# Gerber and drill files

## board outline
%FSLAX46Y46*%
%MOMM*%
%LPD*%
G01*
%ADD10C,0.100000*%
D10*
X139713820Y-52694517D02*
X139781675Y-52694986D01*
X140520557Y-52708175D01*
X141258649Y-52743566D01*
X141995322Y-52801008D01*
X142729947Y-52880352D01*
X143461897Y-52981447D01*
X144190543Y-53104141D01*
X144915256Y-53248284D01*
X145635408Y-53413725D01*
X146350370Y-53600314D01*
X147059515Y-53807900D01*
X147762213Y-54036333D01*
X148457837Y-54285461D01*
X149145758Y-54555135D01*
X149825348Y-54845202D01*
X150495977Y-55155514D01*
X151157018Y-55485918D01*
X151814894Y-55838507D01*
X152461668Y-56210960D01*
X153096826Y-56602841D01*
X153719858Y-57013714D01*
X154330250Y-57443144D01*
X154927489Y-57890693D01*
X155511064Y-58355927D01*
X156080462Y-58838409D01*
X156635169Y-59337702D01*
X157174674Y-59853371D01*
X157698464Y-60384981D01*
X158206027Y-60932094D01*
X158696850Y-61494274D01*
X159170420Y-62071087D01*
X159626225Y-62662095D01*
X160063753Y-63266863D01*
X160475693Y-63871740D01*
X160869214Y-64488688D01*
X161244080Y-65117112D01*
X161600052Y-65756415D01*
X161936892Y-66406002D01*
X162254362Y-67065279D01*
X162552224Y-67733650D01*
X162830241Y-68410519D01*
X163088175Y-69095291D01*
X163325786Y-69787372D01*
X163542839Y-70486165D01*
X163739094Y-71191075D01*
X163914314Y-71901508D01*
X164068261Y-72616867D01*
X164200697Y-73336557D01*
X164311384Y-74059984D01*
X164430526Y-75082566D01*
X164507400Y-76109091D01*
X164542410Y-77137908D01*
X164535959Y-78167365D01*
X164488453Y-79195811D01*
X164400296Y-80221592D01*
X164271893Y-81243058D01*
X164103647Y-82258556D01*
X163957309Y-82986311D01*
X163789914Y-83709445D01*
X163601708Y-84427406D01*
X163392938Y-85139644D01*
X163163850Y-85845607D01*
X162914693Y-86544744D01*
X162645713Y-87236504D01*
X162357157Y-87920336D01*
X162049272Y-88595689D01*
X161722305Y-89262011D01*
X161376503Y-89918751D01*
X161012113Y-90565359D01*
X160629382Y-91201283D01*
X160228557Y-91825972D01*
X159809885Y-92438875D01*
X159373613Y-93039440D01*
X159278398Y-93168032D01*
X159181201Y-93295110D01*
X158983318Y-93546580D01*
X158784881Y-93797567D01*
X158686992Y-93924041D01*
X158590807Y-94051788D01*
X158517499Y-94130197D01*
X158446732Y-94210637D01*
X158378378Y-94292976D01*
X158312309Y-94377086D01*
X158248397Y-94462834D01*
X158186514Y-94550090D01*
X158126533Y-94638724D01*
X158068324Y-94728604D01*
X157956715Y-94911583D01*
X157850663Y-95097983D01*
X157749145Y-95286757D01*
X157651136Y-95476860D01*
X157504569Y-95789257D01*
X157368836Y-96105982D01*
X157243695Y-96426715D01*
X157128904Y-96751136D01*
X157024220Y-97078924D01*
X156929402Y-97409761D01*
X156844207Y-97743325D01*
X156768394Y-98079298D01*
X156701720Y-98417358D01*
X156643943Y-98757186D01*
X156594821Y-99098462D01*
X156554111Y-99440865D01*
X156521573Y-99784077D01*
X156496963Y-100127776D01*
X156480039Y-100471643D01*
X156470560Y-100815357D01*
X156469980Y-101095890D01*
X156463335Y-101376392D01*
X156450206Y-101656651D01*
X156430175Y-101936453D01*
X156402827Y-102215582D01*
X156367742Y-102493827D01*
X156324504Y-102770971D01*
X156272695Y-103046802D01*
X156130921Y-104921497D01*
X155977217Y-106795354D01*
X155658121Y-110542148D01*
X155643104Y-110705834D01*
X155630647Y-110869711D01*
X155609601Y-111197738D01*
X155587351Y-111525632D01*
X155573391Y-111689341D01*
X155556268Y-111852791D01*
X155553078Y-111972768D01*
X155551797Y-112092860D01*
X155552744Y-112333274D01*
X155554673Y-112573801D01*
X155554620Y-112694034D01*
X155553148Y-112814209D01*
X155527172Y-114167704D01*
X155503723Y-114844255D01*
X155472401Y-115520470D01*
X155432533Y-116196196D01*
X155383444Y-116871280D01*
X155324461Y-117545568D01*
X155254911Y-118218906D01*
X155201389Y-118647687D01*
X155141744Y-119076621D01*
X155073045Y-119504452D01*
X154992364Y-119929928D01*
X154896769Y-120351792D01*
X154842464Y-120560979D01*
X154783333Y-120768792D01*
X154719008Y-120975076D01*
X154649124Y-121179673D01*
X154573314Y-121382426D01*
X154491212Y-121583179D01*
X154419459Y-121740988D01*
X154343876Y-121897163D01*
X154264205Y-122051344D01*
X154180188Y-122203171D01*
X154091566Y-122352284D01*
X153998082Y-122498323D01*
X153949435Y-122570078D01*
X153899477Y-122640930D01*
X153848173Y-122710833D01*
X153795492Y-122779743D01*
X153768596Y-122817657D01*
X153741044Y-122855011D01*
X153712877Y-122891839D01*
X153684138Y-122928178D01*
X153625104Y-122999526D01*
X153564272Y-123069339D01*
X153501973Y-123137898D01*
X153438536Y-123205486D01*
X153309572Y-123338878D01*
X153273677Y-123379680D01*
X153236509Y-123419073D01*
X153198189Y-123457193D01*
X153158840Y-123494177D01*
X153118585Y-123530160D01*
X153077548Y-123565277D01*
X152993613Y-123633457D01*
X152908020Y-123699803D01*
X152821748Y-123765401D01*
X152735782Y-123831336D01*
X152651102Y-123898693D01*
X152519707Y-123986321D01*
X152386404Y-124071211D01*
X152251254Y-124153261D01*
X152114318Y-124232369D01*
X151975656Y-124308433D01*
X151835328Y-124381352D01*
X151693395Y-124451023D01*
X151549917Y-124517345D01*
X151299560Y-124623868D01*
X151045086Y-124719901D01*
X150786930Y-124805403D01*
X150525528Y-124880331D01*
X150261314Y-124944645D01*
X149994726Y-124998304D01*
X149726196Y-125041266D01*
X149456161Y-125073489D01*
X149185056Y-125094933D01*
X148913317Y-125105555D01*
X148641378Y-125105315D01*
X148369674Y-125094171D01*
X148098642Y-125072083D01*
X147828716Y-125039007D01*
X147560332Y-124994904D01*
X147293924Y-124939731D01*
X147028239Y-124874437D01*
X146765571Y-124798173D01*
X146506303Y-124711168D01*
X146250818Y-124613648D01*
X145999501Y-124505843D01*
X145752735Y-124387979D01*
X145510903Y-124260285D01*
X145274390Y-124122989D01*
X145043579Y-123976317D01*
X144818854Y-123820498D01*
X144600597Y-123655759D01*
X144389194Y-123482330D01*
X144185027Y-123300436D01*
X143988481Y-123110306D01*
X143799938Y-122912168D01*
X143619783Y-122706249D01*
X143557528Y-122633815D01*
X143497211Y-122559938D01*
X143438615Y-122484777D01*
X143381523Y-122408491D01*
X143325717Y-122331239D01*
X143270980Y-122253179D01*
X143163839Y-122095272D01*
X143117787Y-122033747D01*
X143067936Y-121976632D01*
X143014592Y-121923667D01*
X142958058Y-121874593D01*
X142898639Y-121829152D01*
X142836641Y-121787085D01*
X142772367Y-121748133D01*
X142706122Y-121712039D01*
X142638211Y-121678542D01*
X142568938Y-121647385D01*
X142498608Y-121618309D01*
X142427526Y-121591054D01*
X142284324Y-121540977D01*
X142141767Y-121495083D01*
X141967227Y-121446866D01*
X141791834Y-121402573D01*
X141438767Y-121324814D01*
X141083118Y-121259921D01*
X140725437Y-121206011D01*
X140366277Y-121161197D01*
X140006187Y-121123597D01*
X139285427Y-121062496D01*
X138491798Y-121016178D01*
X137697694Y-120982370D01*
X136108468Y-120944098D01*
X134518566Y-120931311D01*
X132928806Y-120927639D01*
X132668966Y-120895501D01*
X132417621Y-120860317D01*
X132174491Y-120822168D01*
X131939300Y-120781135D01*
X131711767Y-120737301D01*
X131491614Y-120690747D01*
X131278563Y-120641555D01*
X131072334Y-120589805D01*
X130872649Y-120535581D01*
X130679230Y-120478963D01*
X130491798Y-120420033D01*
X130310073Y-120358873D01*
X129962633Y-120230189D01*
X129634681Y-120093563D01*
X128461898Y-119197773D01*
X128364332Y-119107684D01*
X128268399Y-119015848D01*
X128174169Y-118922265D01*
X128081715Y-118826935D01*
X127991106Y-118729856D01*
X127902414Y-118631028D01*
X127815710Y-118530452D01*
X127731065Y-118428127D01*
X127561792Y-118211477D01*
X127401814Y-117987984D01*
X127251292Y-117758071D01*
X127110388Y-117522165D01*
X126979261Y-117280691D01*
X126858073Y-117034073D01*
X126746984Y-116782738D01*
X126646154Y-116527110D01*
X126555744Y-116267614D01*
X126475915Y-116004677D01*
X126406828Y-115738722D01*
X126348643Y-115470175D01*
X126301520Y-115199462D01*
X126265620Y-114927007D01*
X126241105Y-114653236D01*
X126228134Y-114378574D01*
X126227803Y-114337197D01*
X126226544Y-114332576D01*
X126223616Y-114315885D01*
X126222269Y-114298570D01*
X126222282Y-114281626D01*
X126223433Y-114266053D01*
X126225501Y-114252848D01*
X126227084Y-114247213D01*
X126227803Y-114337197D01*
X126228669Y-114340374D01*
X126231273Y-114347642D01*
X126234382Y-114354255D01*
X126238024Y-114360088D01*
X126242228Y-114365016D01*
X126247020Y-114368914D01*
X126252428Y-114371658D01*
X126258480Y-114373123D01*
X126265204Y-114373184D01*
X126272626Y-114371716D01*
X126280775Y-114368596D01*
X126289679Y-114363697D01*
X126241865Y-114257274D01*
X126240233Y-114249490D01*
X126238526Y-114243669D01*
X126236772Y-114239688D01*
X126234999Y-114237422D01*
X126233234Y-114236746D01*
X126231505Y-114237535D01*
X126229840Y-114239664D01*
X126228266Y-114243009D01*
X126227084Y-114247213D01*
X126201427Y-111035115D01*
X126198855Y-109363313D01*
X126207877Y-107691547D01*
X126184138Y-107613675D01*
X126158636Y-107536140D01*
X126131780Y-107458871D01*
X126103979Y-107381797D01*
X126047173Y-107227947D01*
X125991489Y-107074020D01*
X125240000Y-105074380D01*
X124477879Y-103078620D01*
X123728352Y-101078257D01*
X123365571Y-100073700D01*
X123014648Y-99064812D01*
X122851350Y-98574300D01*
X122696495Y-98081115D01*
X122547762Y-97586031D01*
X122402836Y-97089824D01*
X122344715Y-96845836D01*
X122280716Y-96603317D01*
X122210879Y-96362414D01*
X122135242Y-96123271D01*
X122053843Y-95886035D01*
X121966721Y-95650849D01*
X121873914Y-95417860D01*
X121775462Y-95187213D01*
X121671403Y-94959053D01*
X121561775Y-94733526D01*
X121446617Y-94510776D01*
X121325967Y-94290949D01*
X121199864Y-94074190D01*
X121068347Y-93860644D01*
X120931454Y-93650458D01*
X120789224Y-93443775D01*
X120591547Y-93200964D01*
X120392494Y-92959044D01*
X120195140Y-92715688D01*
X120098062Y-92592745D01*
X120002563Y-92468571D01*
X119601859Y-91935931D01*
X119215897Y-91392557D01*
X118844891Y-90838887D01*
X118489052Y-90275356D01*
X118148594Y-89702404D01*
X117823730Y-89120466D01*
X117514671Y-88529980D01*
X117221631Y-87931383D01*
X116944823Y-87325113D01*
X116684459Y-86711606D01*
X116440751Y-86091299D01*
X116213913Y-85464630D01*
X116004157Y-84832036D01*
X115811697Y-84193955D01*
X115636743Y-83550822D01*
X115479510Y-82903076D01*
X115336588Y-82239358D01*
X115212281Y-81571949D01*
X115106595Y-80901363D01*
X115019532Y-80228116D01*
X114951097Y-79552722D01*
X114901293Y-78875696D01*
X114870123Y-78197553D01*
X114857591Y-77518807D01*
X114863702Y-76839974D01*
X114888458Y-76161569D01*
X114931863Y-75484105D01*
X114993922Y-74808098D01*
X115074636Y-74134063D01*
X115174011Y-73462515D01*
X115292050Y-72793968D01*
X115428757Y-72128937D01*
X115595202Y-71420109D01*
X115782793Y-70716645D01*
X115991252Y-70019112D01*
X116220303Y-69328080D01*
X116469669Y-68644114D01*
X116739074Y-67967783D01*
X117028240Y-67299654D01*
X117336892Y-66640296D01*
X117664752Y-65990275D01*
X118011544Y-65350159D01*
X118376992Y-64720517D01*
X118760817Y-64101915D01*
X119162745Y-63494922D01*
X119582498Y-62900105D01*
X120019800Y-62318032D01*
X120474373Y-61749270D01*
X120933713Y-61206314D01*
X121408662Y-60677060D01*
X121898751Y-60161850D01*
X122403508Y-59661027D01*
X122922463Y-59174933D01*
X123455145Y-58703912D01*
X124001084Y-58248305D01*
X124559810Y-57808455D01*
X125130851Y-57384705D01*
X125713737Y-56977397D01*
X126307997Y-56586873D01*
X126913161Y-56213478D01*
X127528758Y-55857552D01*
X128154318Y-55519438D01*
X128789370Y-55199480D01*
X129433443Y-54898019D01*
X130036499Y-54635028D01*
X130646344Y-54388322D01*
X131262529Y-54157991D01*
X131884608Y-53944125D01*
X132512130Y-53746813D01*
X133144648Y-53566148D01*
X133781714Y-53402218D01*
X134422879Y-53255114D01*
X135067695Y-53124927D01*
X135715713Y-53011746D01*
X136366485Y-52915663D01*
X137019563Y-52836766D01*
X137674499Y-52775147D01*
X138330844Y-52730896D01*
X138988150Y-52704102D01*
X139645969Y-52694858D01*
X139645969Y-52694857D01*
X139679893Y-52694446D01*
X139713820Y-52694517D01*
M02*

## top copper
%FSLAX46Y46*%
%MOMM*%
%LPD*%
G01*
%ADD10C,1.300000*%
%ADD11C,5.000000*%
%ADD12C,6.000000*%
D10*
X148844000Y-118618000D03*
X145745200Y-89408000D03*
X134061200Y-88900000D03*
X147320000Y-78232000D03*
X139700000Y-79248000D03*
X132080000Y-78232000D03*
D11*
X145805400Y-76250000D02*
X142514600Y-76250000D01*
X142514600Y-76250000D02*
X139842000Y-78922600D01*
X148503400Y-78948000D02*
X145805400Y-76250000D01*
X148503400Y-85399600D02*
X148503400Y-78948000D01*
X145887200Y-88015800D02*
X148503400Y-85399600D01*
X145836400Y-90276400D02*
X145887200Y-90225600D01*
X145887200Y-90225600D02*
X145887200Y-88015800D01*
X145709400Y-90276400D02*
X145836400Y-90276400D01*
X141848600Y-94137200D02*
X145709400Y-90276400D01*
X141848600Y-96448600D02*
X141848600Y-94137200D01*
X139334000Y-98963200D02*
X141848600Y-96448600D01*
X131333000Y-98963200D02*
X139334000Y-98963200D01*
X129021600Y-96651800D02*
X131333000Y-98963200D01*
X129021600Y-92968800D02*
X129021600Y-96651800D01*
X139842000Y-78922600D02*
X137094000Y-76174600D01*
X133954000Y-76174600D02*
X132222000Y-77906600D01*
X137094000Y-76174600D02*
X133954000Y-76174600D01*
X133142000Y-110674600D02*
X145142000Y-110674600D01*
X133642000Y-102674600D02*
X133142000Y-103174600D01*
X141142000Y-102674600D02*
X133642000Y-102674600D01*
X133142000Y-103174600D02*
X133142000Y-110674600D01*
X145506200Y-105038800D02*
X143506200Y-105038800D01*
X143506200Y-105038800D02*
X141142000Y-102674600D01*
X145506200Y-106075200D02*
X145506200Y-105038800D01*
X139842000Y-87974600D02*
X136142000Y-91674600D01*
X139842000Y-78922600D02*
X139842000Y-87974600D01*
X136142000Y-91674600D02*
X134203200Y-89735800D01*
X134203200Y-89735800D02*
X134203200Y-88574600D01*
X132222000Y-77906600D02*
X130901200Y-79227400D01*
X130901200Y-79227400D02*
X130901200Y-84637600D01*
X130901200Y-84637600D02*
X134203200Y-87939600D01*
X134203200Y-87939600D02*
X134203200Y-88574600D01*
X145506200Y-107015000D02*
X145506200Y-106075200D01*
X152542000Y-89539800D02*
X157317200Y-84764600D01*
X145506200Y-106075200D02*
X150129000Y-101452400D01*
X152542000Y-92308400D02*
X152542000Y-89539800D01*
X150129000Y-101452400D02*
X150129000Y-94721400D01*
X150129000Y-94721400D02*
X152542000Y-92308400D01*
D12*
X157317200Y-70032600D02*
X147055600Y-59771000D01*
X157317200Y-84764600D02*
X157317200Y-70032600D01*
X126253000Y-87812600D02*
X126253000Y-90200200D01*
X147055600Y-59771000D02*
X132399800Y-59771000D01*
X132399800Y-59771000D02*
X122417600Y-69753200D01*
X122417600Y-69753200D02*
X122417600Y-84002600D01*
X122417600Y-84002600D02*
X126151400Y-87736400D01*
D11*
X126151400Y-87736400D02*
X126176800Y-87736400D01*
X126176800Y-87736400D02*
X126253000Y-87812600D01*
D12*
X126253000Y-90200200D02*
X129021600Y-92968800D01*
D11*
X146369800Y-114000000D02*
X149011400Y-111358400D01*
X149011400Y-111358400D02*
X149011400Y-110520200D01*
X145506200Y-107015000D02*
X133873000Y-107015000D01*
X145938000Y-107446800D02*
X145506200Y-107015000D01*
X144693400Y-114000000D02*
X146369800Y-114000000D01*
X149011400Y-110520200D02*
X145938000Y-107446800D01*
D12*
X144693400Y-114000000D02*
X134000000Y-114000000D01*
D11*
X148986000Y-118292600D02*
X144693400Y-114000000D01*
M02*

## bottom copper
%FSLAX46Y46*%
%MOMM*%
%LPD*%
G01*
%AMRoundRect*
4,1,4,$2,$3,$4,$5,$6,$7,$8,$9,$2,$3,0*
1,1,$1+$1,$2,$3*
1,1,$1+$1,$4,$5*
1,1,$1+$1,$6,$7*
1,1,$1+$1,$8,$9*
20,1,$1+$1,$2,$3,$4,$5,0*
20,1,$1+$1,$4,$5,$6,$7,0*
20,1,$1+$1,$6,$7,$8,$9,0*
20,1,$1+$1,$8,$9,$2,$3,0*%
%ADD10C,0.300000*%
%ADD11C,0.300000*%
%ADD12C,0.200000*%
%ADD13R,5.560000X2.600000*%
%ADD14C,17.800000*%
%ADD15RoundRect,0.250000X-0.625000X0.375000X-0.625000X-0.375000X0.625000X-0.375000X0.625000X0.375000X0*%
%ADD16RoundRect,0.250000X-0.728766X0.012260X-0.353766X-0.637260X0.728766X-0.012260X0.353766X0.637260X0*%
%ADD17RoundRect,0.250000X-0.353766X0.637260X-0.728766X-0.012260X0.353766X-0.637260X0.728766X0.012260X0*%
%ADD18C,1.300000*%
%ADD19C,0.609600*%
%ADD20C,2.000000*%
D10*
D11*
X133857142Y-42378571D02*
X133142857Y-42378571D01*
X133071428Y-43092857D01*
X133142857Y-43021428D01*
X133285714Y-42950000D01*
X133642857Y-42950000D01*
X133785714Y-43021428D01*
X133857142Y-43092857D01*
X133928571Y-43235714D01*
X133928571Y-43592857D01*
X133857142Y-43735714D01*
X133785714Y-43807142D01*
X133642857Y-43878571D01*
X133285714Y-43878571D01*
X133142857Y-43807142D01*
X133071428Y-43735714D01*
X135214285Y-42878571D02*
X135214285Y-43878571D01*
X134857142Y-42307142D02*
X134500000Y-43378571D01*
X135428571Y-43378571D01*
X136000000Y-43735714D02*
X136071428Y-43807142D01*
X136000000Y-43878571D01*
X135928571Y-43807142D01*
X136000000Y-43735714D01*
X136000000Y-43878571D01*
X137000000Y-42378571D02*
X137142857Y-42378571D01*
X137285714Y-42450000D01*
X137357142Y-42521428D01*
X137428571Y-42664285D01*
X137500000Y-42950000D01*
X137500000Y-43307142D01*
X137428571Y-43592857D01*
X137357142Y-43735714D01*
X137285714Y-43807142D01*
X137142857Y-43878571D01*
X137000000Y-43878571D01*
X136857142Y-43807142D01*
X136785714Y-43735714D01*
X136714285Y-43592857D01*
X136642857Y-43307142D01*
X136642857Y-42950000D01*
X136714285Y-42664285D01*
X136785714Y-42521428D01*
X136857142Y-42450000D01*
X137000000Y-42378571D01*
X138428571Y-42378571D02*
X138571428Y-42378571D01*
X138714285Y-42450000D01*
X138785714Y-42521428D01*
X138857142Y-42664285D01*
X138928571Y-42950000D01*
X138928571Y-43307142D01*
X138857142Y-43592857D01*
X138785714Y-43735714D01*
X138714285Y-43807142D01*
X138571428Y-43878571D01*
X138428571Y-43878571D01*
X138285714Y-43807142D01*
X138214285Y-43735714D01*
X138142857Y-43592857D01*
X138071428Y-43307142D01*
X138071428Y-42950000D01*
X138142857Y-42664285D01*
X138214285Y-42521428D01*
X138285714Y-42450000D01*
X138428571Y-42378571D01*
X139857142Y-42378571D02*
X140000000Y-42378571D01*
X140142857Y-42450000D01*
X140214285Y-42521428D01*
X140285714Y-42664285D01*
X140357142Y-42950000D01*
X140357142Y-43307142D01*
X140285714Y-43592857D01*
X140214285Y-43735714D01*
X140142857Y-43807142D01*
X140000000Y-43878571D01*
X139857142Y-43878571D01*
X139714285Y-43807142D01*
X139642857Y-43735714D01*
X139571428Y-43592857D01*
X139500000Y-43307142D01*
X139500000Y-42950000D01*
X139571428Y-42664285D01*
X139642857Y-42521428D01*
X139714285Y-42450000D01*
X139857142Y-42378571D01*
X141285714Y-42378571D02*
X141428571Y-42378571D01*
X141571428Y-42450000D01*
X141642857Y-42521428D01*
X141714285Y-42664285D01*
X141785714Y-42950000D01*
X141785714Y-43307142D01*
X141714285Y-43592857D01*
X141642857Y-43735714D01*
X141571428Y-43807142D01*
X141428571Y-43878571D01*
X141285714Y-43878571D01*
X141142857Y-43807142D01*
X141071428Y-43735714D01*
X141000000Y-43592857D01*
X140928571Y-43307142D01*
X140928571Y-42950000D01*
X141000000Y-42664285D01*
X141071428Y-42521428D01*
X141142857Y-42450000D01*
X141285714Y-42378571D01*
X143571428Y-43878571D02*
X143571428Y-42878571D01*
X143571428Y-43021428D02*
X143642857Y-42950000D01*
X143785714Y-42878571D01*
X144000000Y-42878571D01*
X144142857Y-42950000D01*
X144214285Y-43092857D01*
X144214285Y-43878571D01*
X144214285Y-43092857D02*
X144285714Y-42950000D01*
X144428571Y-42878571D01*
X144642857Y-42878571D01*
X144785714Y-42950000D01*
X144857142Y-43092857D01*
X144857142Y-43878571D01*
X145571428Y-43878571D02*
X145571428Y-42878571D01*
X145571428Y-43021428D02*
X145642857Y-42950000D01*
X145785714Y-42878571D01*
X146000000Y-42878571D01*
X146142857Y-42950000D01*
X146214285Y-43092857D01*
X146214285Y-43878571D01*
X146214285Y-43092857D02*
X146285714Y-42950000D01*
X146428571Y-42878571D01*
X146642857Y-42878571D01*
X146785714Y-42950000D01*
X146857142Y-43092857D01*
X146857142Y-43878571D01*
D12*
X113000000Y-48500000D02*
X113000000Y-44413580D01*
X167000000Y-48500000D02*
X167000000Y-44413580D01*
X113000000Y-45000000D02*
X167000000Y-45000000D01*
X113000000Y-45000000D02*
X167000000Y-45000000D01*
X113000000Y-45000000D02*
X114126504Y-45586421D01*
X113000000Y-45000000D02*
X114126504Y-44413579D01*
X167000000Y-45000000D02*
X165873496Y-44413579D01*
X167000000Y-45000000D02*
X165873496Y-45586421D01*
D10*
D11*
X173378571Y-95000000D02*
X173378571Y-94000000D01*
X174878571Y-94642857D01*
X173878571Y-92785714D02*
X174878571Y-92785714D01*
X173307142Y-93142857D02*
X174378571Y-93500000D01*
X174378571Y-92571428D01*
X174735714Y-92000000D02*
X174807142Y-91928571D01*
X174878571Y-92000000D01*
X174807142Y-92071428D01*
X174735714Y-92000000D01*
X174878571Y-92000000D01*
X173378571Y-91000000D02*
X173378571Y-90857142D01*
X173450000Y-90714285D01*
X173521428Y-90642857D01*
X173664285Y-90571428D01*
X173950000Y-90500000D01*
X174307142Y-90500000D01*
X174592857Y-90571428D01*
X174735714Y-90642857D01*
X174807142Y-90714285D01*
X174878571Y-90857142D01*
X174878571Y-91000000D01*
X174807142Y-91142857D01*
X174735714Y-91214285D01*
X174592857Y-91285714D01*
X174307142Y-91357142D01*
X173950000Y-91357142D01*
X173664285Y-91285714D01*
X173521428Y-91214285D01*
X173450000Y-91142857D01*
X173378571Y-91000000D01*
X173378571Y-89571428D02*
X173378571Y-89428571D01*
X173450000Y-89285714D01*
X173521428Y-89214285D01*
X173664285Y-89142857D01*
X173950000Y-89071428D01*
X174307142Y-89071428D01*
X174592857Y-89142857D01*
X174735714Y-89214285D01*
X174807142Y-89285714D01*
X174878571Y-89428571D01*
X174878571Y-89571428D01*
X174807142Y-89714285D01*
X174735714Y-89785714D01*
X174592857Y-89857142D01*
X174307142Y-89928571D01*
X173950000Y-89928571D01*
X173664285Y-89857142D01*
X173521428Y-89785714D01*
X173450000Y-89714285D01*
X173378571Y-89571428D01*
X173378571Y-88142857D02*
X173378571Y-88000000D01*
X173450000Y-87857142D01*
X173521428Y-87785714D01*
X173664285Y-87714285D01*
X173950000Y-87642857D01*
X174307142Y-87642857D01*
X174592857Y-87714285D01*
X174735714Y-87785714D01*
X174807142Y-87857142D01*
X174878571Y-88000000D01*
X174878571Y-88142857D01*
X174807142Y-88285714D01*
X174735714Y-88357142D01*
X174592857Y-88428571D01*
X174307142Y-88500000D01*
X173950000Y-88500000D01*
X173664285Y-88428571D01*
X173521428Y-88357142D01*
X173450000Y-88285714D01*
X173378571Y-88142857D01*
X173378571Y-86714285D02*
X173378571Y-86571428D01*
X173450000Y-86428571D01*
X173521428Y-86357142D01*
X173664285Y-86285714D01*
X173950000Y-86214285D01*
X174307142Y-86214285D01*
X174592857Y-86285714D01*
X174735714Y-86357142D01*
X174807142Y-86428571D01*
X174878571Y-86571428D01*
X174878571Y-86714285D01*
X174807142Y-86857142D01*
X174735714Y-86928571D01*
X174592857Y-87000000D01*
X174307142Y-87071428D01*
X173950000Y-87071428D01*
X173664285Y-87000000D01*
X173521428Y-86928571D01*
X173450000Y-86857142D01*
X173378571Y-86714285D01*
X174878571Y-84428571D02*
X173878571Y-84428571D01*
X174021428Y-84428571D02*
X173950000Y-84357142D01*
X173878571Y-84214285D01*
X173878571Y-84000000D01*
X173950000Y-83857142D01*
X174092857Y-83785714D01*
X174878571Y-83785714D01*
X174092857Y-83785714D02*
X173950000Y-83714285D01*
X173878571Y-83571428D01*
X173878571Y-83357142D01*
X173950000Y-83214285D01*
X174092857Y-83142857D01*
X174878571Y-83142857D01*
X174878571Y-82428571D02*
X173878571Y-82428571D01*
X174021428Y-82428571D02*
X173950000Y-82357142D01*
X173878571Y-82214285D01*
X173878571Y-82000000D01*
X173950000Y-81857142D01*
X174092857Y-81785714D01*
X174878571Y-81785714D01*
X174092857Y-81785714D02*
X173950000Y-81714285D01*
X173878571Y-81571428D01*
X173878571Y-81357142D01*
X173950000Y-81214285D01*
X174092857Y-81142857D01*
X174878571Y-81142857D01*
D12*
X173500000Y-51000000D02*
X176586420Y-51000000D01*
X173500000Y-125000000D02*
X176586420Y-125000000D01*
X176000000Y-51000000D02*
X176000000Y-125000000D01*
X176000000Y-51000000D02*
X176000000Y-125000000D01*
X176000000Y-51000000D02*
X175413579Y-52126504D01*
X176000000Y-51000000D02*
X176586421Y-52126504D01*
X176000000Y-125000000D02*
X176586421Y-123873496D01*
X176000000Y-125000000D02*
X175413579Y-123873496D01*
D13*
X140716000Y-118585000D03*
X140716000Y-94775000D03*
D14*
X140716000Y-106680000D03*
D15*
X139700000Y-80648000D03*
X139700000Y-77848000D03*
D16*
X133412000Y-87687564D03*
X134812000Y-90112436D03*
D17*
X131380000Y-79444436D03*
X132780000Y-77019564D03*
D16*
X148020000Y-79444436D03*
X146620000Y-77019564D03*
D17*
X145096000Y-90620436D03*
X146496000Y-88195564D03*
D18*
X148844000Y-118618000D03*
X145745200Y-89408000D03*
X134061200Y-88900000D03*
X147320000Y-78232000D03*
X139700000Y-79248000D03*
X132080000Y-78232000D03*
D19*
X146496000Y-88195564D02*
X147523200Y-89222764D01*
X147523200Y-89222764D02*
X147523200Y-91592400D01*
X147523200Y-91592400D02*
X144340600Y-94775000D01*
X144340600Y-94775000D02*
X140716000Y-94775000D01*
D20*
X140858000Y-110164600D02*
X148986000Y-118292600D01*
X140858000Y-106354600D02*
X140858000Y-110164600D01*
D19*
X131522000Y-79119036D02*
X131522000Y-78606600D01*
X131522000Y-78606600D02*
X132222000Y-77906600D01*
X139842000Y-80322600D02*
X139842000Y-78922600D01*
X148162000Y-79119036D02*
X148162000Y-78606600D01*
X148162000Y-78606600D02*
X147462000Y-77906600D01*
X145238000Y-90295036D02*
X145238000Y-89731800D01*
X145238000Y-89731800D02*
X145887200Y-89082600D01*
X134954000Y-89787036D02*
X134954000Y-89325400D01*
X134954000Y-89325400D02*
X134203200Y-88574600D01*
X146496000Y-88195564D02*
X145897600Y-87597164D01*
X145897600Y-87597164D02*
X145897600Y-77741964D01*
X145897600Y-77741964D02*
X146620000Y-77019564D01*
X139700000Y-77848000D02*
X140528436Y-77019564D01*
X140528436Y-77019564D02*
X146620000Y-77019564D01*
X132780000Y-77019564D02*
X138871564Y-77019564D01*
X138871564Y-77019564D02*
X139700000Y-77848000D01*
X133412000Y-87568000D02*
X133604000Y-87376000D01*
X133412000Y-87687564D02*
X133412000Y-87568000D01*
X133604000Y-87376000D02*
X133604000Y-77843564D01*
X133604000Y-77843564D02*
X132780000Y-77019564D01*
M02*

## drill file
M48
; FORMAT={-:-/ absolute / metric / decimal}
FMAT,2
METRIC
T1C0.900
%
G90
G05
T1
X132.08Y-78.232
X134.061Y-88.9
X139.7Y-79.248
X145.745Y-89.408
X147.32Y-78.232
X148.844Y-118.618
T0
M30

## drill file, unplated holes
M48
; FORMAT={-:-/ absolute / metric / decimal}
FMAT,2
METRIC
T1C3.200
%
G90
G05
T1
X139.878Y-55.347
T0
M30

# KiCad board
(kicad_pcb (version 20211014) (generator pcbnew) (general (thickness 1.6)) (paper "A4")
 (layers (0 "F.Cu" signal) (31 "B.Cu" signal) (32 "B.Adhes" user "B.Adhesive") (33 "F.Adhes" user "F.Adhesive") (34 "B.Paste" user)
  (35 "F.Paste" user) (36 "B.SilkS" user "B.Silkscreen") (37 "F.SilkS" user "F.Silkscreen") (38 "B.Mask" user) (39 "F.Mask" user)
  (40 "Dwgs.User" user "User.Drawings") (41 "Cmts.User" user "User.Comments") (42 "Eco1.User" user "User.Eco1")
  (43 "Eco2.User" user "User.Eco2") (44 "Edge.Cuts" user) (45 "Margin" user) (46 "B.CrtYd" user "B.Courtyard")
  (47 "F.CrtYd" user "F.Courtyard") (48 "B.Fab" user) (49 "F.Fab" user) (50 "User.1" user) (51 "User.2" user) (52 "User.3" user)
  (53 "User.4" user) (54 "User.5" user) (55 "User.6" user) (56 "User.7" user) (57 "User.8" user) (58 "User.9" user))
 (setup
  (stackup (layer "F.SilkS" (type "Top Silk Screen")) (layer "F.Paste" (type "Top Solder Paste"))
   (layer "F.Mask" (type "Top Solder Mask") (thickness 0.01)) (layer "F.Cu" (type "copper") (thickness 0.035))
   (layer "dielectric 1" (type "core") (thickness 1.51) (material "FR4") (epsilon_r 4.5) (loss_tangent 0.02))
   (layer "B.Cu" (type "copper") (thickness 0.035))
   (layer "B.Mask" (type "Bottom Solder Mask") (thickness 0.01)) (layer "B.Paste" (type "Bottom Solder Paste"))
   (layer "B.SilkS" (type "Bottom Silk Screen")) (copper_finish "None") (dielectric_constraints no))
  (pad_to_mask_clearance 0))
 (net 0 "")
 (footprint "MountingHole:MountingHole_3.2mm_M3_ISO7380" (layer "F.Cu") (at 139.8778 55.3466)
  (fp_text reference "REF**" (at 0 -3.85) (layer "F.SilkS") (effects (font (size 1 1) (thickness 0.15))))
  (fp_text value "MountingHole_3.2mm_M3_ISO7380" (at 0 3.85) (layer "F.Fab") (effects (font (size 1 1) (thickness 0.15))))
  (pad "" np_thru_hole circle (at 0 0) (size 3.2 3.2) (drill 3.2) (layers *.Cu *.Mask)))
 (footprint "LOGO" (layer "F.Cu") (at 139.7 88.9)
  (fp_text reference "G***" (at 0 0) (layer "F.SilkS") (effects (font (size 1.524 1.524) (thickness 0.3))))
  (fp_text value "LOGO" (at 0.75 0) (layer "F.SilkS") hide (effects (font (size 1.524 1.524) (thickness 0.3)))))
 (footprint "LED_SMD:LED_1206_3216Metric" (layer "B.Cu") (at 139.7 79.248 -90)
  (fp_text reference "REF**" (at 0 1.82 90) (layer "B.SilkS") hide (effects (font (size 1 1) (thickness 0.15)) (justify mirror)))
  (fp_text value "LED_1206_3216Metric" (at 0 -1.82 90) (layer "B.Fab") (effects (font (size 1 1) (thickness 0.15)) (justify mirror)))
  (pad "1" smd roundrect (at -1.4 0 270) (size 1.25 1.75) (layers "B.Cu" "B.Paste" "B.Mask") (roundrect_rratio 0.2))
  (pad "2" smd roundrect (at 1.4 0 270) (size 1.25 1.75) (layers "B.Cu" "B.Paste" "B.Mask") (roundrect_rratio 0.2)))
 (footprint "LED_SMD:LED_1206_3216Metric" (layer "B.Cu") (at 147.32 78.232 -60)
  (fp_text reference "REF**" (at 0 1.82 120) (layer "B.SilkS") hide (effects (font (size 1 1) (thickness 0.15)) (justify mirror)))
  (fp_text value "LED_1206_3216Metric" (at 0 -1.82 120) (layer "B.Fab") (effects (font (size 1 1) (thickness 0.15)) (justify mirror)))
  (pad "1" smd roundrect (at -1.4 0 300) (size 1.25 1.75) (layers "B.Cu" "B.Paste" "B.Mask") (roundrect_rratio 0.2))
  (pad "2" smd roundrect (at 1.4 0 300) (size 1.25 1.75) (layers "B.Cu" "B.Paste" "B.Mask") (roundrect_rratio 0.2)))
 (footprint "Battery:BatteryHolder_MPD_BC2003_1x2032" (layer "B.Cu") (at 140.716 106.68 90)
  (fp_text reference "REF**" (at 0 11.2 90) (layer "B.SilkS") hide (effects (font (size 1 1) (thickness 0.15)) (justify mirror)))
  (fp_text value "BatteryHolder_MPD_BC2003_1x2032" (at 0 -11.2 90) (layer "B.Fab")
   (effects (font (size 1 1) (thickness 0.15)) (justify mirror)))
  (pad "1" smd rect (at 11.905 0 90) (size 2.6 5.56) (layers "B.Cu" "B.Paste" "B.Mask"))
  (pad "1" smd rect (at -11.905 0 90) (size 2.6 5.56) (layers "B.Cu" "B.Paste" "B.Mask"))
  (pad "2" smd circle (at 0 0 90) (size 17.8 17.8) (layers "B.Cu" "B.Mask")))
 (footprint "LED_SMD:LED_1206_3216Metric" (layer "B.Cu") (at 132.08 78.232 -120)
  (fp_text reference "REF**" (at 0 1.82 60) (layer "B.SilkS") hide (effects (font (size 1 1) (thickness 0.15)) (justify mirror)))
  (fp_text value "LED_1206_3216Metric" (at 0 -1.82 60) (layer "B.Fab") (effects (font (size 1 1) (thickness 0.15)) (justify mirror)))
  (pad "1" smd roundrect (at -1.4 0 240) (size 1.25 1.75) (layers "B.Cu" "B.Paste" "B.Mask") (roundrect_rratio 0.2))
  (pad "2" smd roundrect (at 1.4 0 240) (size 1.25 1.75) (layers "B.Cu" "B.Paste" "B.Mask") (roundrect_rratio 0.2)))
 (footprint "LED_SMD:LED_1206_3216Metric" (layer "B.Cu") (at 134.112 88.9 -60)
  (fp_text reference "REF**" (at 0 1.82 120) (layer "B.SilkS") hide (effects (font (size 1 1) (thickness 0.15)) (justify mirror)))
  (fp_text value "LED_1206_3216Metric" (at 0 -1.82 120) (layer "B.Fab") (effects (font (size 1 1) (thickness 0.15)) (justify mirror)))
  (pad "1" smd roundrect (at -1.4 0 300) (size 1.25 1.75) (layers "B.Cu" "B.Paste" "B.Mask") (roundrect_rratio 0.2))
  (pad "2" smd roundrect (at 1.4 0 300) (size 1.25 1.75) (layers "B.Cu" "B.Paste" "B.Mask") (roundrect_rratio 0.2)))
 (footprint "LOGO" (layer "B.Cu") (at 139.7 88.9 180)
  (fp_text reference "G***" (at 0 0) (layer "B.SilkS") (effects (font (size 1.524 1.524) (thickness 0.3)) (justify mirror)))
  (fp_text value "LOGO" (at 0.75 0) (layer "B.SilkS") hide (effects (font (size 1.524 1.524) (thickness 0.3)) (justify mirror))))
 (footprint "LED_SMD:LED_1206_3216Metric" (layer "B.Cu") (at 145.796 89.408 -120)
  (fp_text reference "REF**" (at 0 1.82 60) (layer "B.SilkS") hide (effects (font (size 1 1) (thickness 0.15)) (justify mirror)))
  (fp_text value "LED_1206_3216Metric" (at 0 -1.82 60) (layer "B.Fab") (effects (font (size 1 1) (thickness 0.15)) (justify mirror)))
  (pad "1" smd roundrect (at -1.4 0 240) (size 1.25 1.75) (layers "B.Cu" "B.Paste" "B.Mask") (roundrect_rratio 0.2))
  (pad "2" smd roundrect (at 1.4 0 240) (size 1.25 1.75) (layers "B.Cu" "B.Paste" "B.Mask") (roundrect_rratio 0.2)))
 (gr_poly
  (pts (xy 139.71382 52.694517) (xy 139.781675 52.694986) (xy 140.520557 52.708175) (xy 141.258649 52.743566) (xy 141.995322 52.801008)
   (xy 142.729947 52.880352) (xy 143.461897 52.981447) (xy 144.190543 53.104141) (xy 144.915256 53.248284) (xy 145.635408 53.413725)
   (xy 146.35037 53.600314) (xy 147.059515 53.8079) (xy 147.762213 54.036333) (xy 148.457837 54.285461) (xy 149.145758 54.555135)
   (xy 149.825348 54.845202) (xy 150.495977 55.155514) (xy 151.157018 55.485918) (xy 151.814894 55.838507) (xy 152.461668 56.21096)
   (xy 153.096826 56.602841) (xy 153.719858 57.013714) (xy 154.33025 57.443144) (xy 154.927489 57.890693) (xy 155.511064 58.355927)
   (xy 156.080462 58.838409) (xy 156.635169 59.337702) (xy 157.174674 59.853371) (xy 157.698464 60.384981) (xy 158.206027 60.932094)
   (xy 158.69685 61.494274) (xy 159.17042 62.071087) (xy 159.626225 62.662095) (xy 160.063753 63.266863) (xy 160.475693 63.87174)
   (xy 160.869214 64.488688) (xy 161.24408 65.117112) (xy 161.600052 65.756415) (xy 161.936892 66.406002) (xy 162.254362 67.065279)
   (xy 162.552224 67.73365) (xy 162.830241 68.410519) (xy 163.088175 69.095291) (xy 163.325786 69.787372) (xy 163.542839 70.486165)
   (xy 163.739094 71.191075) (xy 163.914314 71.901508) (xy 164.068261 72.616867) (xy 164.200697 73.336557) (xy 164.311384 74.059984)
   (xy 164.430526 75.082566) (xy 164.5074 76.109091) (xy 164.54241 77.137908) (xy 164.535959 78.167365) (xy 164.488453 79.195811)
   (xy 164.400296 80.221592) (xy 164.271893 81.243058) (xy 164.103647 82.258556) (xy 163.957309 82.986311) (xy 163.789914 83.709445)
   (xy 163.601708 84.427406) (xy 163.392938 85.139644) (xy 163.16385 85.845607) (xy 162.914693 86.544744) (xy 162.645713 87.236504)
   (xy 162.357157 87.920336) (xy 162.049272 88.595689) (xy 161.722305 89.262011) (xy 161.376503 89.918751) (xy 161.012113 90.565359)
   (xy 160.629382 91.201283) (xy 160.228557 91.825972) (xy 159.809885 92.438875) (xy 159.373613 93.03944) (xy 159.278398 93.168032)
   (xy 159.181201 93.29511) (xy 158.983318 93.54658) (xy 158.784881 93.797567) (xy 158.686992 93.924041) (xy 158.590807 94.051788)
   (xy 158.517499 94.130197) (xy 158.446732 94.210637) (xy 158.378378 94.292976) (xy 158.312309 94.377086) (xy 158.248397 94.462834)
   (xy 158.186514 94.55009) (xy 158.126533 94.638724) (xy 158.068324 94.728604) (xy 157.956715 94.911583) (xy 157.850663 95.097983)
   (xy 157.749145 95.286757) (xy 157.651136 95.47686) (xy 157.504569 95.789257) (xy 157.368836 96.105982) (xy 157.243695 96.426715)
   (xy 157.128904 96.751136) (xy 157.02422 97.078924) (xy 156.929402 97.409761) (xy 156.844207 97.743325) (xy 156.768394 98.079298)
   (xy 156.70172 98.417358) (xy 156.643943 98.757186) (xy 156.594821 99.098462) (xy 156.554111 99.440865) (xy 156.521573 99.784077)
   (xy 156.496963 100.127776) (xy 156.480039 100.471643) (xy 156.47056 100.815357) (xy 156.46998 101.09589) (xy 156.463335 101.376392)
   (xy 156.450206 101.656651) (xy 156.430175 101.936453) (xy 156.402827 102.215582) (xy 156.367742 102.493827) (xy 156.324504 102.770971)
   (xy 156.272695 103.046802) (xy 156.130921 104.921497) (xy 155.977217 106.795354) (xy 155.658121 110.542148) (xy 155.643104 110.705834)
   (xy 155.630647 110.869711) (xy 155.609601 111.197738) (xy 155.587351 111.525632) (xy 155.573391 111.689341) (xy 155.556268 111.852791)
   (xy 155.553078 111.972768) (xy 155.551797 112.09286) (xy 155.552744 112.333274) (xy 155.554673 112.573801) (xy 155.55462 112.694034)
   (xy 155.553148 112.814209) (xy 155.527172 114.167704) (xy 155.503723 114.844255) (xy 155.472401 115.52047) (xy 155.432533 116.196196)
   (xy 155.383444 116.87128) (xy 155.324461 117.545568) (xy 155.254911 118.218906) (xy 155.201389 118.647687) (xy 155.141744 119.076621)
   (xy 155.073045 119.504452) (xy 154.992364 119.929928) (xy 154.896769 120.351792) (xy 154.842464 120.560979) (xy 154.783333 120.768792)
   (xy 154.719008 120.975076) (xy 154.649124 121.179673) (xy 154.573314 121.382426) (xy 154.491212 121.583179) (xy 154.419459 121.740988)
   (xy 154.343876 121.897163) (xy 154.264205 122.051344) (xy 154.180188 122.203171) (xy 154.091566 122.352284) (xy 153.998082 122.498323)
   (xy 153.949435 122.570078) (xy 153.899477 122.64093) (xy 153.848173 122.710833) (xy 153.795492 122.779743) (xy 153.768596 122.817657)
   (xy 153.741044 122.855011) (xy 153.712877 122.891839) (xy 153.684138 122.928178) (xy 153.625104 122.999526) (xy 153.564272 123.069339)
   (xy 153.501973 123.137898) (xy 153.438536 123.205486) (xy 153.309572 123.338878) (xy 153.273677 123.37968) (xy 153.236509 123.419073)
   (xy 153.198189 123.457193) (xy 153.15884 123.494177) (xy 153.118585 123.53016) (xy 153.077548 123.565277) (xy 152.993613 123.633457)
   (xy 152.90802 123.699803) (xy 152.821748 123.765401) (xy 152.735782 123.831336) (xy 152.651102 123.898693) (xy 152.519707 123.986321)
   (xy 152.386404 124.071211) (xy 152.251254 124.153261) (xy 152.114318 124.232369) (xy 151.975656 124.308433) (xy 151.835328 124.381352)
   (xy 151.693395 124.451023) (xy 151.549917 124.517345) (xy 151.29956 124.623868) (xy 151.045086 124.719901) (xy 150.78693 124.805403)
   (xy 150.525528 124.880331) (xy 150.261314 124.944645) (xy 149.994726 124.998304) (xy 149.726196 125.041266) (xy 149.456161 125.073489)
   (xy 149.185056 125.094933) (xy 148.913317 125.105555) (xy 148.641378 125.105315) (xy 148.369674 125.094171) (xy 148.098642 125.072083)
   (xy 147.828716 125.039007) (xy 147.560332 124.994904) (xy 147.293924 124.939731) (xy 147.028239 124.874437) (xy 146.765571 124.798173)
   (xy 146.506303 124.711168) (xy 146.250818 124.613648) (xy 145.999501 124.505843) (xy 145.752735 124.387979) (xy 145.510903 124.260285)
   (xy 145.27439 124.122989) (xy 145.043579 123.976317) (xy 144.818854 123.820498) (xy 144.600597 123.655759) (xy 144.389194 123.48233)
   (xy 144.185027 123.300436) (xy 143.988481 123.110306) (xy 143.799938 122.912168) (xy 143.619783 122.706249) (xy 143.557528 122.633815)
   (xy 143.497211 122.559938) (xy 143.438615 122.484777) (xy 143.381523 122.408491) (xy 143.325717 122.331239) (xy 143.27098 122.253179)
   (xy 143.163839 122.095272) (xy 143.117787 122.033747) (xy 143.067936 121.976632) (xy 143.014592 121.923667) (xy 142.958058 121.874593)
   (xy 142.898639 121.829152) (xy 142.836641 121.787085) (xy 142.772367 121.748133) (xy 142.706122 121.712039) (xy 142.638211 121.678542)
   (xy 142.568938 121.647385) (xy 142.498608 121.618309) (xy 142.427526 121.591054) (xy 142.284324 121.540977) (xy 142.141767 121.495083)
   (xy 141.967227 121.446866) (xy 141.791834 121.402573) (xy 141.438767 121.324814) (xy 141.083118 121.259921) (xy 140.725437 121.206011)
   (xy 140.366277 121.161197) (xy 140.006187 121.123597) (xy 139.285427 121.062496) (xy 138.491798 121.016178) (xy 137.697694 120.98237)
   (xy 136.108468 120.944098) (xy 134.518566 120.931311) (xy 132.928806 120.927639) (xy 132.668966 120.895501) (xy 132.417621 120.860317)
   (xy 132.174491 120.822168) (xy 131.9393 120.781135) (xy 131.711767 120.737301) (xy 131.491614 120.690747) (xy 131.278563 120.641555)
   (xy 131.072334 120.589805) (xy 130.872649 120.535581) (xy 130.67923 120.478963) (xy 130.491798 120.420033) (xy 130.310073 120.358873)
   (xy 129.962633 120.230189) (xy 129.634681 120.093563) (xy 128.461898 119.197773) (xy 128.364332 119.107684) (xy 128.268399 119.015848)
   (xy 128.174169 118.922265) (xy 128.081715 118.826935) (xy 127.991106 118.729856) (xy 127.902414 118.631028) (xy 127.81571 118.530452)
   (xy 127.731065 118.428127) (xy 127.561792 118.211477) (xy 127.401814 117.987984) (xy 127.251292 117.758071) (xy 127.110388 117.522165)
   (xy 126.979261 117.280691) (xy 126.858073 117.034073) (xy 126.746984 116.782738) (xy 126.646154 116.52711) (xy 126.555744 116.267614)
   (xy 126.475915 116.004677) (xy 126.406828 115.738722) (xy 126.348643 115.470175) (xy 126.30152 115.199462) (xy 126.26562 114.927007)
   (xy 126.241105 114.653236) (xy 126.228134 114.378574) (xy 126.227803 114.337197) (xy 126.226544 114.332576) (xy 126.223616 114.315885)
   (xy 126.222269 114.29857) (xy 126.222282 114.281626) (xy 126.223433 114.266053) (xy 126.225501 114.252848) (xy 126.227084 114.247213)
   (xy 126.227803 114.337197) (xy 126.228669 114.340374) (xy 126.231273 114.347642) (xy 126.234382 114.354255) (xy 126.238024 114.360088)
   (xy 126.242228 114.365016) (xy 126.24702 114.368914) (xy 126.252428 114.371658) (xy 126.25848 114.373123) (xy 126.265204 114.373184)
   (xy 126.272626 114.371716) (xy 126.280775 114.368596) (xy 126.289679 114.363697) (xy 126.241865 114.257274) (xy 126.240233 114.24949)
   (xy 126.238526 114.243669) (xy 126.236772 114.239688) (xy 126.234999 114.237422) (xy 126.233234 114.236746) (xy 126.231505 114.237535)
   (xy 126.22984 114.239664) (xy 126.228266 114.243009) (xy 126.227084 114.247213) (xy 126.201427 111.035115) (xy 126.198855 109.363313)
   (xy 126.207877 107.691547) (xy 126.184138 107.613675) (xy 126.158636 107.53614) (xy 126.13178 107.458871) (xy 126.103979 107.381797)
   (xy 126.047173 107.227947) (xy 125.991489 107.07402) (xy 125.24 105.07438) (xy 124.477879 103.07862) (xy 123.728352 101.078257)
   (xy 123.365571 100.0737) (xy 123.014648 99.064812) (xy 122.85135 98.5743) (xy 122.696495 98.081115) (xy 122.547762 97.586031)
   (xy 122.402836 97.089824) (xy 122.344715 96.845836) (xy 122.280716 96.603317) (xy 122.210879 96.362414) (xy 122.135242 96.123271)
   (xy 122.053843 95.886035) (xy 121.966721 95.650849) (xy 121.873914 95.41786) (xy 121.775462 95.187213) (xy 121.671403 94.959053)
   (xy 121.561775 94.733526) (xy 121.446617 94.510776) (xy 121.325967 94.290949) (xy 121.199864 94.07419) (xy 121.068347 93.860644)
   (xy 120.931454 93.650458) (xy 120.789224 93.443775) (xy 120.591547 93.200964) (xy 120.392494 92.959044) (xy 120.19514 92.715688)
   (xy 120.098062 92.592745) (xy 120.002563 92.468571) (xy 119.601859 91.935931) (xy 119.215897 91.392557) (xy 118.844891 90.838887)
   (xy 118.489052 90.275356) (xy 118.148594 89.702404) (xy 117.82373 89.120466) (xy 117.514671 88.52998) (xy 117.221631 87.931383)
   (xy 116.944823 87.325113) (xy 116.684459 86.711606) (xy 116.440751 86.091299) (xy 116.213913 85.46463) (xy 116.004157 84.832036)
   (xy 115.811697 84.193955) (xy 115.636743 83.550822) (xy 115.47951 82.903076) (xy 115.336588 82.239358) (xy 115.212281 81.571949)
   (xy 115.106595 80.901363) (xy 115.019532 80.228116) (xy 114.951097 79.552722) (xy 114.901293 78.875696) (xy 114.870123 78.197553)
   (xy 114.857591 77.518807) (xy 114.863702 76.839974) (xy 114.888458 76.161569) (xy 114.931863 75.484105) (xy 114.993922 74.808098)
   (xy 115.074636 74.134063) (xy 115.174011 73.462515) (xy 115.29205 72.793968) (xy 115.428757 72.128937) (xy 115.595202 71.420109)
   (xy 115.782793 70.716645) (xy 115.991252 70.019112) (xy 116.220303 69.32808) (xy 116.469669 68.644114) (xy 116.739074 67.967783)
   (xy 117.02824 67.299654) (xy 117.336892 66.640296) (xy 117.664752 65.990275) (xy 118.011544 65.350159) (xy 118.376992 64.720517)
   (xy 118.760817 64.101915) (xy 119.162745 63.494922) (xy 119.582498 62.900105) (xy 120.0198 62.318032) (xy 120.474373 61.74927)
   (xy 120.933713 61.206314) (xy 121.408662 60.67706) (xy 121.898751 60.16185) (xy 122.403508 59.661027) (xy 122.922463 59.174933)
   (xy 123.455145 58.703912) (xy 124.001084 58.248305) (xy 124.55981 57.808455) (xy 125.130851 57.384705) (xy 125.713737 56.977397)
   (xy 126.307997 56.586873) (xy 126.913161 56.213478) (xy 127.528758 55.857552) (xy 128.154318 55.519438) (xy 128.78937 55.19948)
   (xy 129.433443 54.898019) (xy 130.036499 54.635028) (xy 130.646344 54.388322) (xy 131.262529 54.157991) (xy 131.884608 53.944125)
   (xy 132.51213 53.746813) (xy 133.144648 53.566148) (xy 133.781714 53.402218) (xy 134.422879 53.255114) (xy 135.067695 53.124927)
   (xy 135.715713 53.011746) (xy 136.366485 52.915663) (xy 137.019563 52.836766) (xy 137.674499 52.775147) (xy 138.330844 52.730896)
   (xy 138.98815 52.704102) (xy 139.645969 52.694858) (xy 139.645969 52.694857) (xy 139.679893 52.694446))
  (layer "Edge.Cuts") (width 0.1) (fill none))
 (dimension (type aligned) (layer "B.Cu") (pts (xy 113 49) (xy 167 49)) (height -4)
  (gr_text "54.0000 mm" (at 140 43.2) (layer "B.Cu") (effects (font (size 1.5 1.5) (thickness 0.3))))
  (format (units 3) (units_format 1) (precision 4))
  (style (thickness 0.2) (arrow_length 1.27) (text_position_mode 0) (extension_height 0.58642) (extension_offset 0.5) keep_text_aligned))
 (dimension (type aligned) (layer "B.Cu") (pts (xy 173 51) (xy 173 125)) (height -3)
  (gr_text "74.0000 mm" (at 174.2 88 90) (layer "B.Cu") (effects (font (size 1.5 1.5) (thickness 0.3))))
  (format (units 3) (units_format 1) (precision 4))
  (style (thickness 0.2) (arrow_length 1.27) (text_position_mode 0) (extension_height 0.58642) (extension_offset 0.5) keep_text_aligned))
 (segment (start 145.5062 107.015) (end 133.873 107.015) (width 5) (layer "F.Cu") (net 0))
 (segment (start 145.7094 90.2764) (end 145.8364 90.2764) (width 5) (layer "F.Cu") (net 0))
 (segment (start 122.4176 84.0026) (end 126.1514 87.7364) (width 6) (layer "F.Cu") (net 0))
 (segment (start 145.8872 88.0158) (end 148.5034 85.3996) (width 5) (layer "F.Cu") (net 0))
 (segment (start 145.8364 90.2764) (end 145.8872 90.2256) (width 5) (layer "F.Cu") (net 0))
 (segment (start 145.5062 105.0388) (end 143.5062 105.0388) (width 5) (layer "F.Cu") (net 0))
 (segment (start 132.222 77.9066) (end 130.9012 79.2274) (width 5) (layer "F.Cu") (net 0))
 (segment (start 130.9012 79.2274) (end 130.9012 84.6376) (width 5) (layer "F.Cu") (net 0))
 (segment (start 139.334 98.9632) (end 141.8486 96.4486) (width 5) (layer "F.Cu") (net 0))
 (segment (start 139.842 87.9746) (end 136.142 91.6746) (width 5) (layer "F.Cu") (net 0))
 (segment (start 129.0216 96.6518) (end 131.333 98.9632) (width 5) (layer "F.Cu") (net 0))
 (segment (start 157.3172 70.0326) (end 147.0556 59.771) (width 6) (layer "F.Cu") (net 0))
 (segment (start 146.3698 114) (end 149.0114 111.3584) (width 5) (layer "F.Cu") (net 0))
 (segment (start 150.129 101.4524) (end 150.129 94.7214) (width 5) (layer "F.Cu") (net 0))
 (segment (start 149.0114 110.5202) (end 145.938 107.4468) (width 5) (layer "F.Cu") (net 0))
 (segment (start 141.8486 94.1372) (end 145.7094 90.2764) (width 5) (layer "F.Cu") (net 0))
 (segment (start 148.986 118.2926) (end 144.6934 114) (width 5) (layer "F.Cu") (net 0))
 (segment (start 122.4176 69.7532) (end 122.4176 84.0026) (width 6) (layer "F.Cu") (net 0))
 (segment (start 152.542 89.5398) (end 157.3172 84.7646) (width 5) (layer "F.Cu") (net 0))
 (segment (start 145.8872 90.2256) (end 145.8872 88.0158) (width 5) (layer "F.Cu") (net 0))
 (segment (start 134.2032 89.7358) (end 134.2032 88.5746) (width 5) (layer "F.Cu") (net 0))
 (segment (start 145.5062 106.0752) (end 145.5062 105.0388) (width 5) (layer "F.Cu") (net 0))
 (segment (start 145.8054 76.25) (end 142.5146 76.25) (width 5) (layer "F.Cu") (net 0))
 (segment (start 133.642 102.6746) (end 133.142 103.1746) (width 5) (layer "F.Cu") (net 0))
 (segment (start 145.938 107.4468) (end 145.5062 107.015) (width 5) (layer "F.Cu") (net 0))
 (segment (start 149.0114 111.3584) (end 149.0114 110.5202) (width 5) (layer "F.Cu") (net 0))
 (segment (start 139.842 78.9226) (end 137.094 76.1746) (width 5) (layer "F.Cu") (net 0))
 (segment (start 141.142 102.6746) (end 133.642 102.6746) (width 5) (layer "F.Cu") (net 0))
 (segment (start 143.5062 105.0388) (end 141.142 102.6746) (width 5) (layer "F.Cu") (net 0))
 (segment (start 139.842 78.9226) (end 139.842 87.9746) (width 5) (layer "F.Cu") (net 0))
 (segment (start 136.142 91.6746) (end 134.2032 89.7358) (width 5) (layer "F.Cu") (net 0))
 (segment (start 134.2032 87.9396) (end 134.2032 88.5746) (width 5) (layer "F.Cu") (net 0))
 (segment (start 142.5146 76.25) (end 139.842 78.9226) (width 5) (layer "F.Cu") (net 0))
 (segment (start 131.333 98.9632) (end 139.334 98.9632) (width 5) (layer "F.Cu") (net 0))
 (segment (start 133.954 76.1746) (end 132.222 77.9066) (width 5) (layer "F.Cu") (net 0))
 (segment (start 152.542 92.3084) (end 152.542 89.5398) (width 5) (layer "F.Cu") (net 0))
 (segment (start 126.253 90.2002) (end 129.0216 92.9688) (width 6) (layer "F.Cu") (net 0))
 (segment (start 150.129 94.7214) (end 152.542 92.3084) (width 5) (layer "F.Cu") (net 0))
 (segment (start 144.6934 114) (end 146.3698 114) (width 5) (layer "F.Cu") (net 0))
 (segment (start 126.253 87.8126) (end 126.253 90.2002) (width 6) (layer "F.Cu") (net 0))
 (segment (start 145.5062 106.0752) (end 150.129 101.4524) (width 5) (layer "F.Cu") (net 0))
 (segment (start 141.8486 96.4486) (end 141.8486 94.1372) (width 5) (layer "F.Cu") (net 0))
 (segment (start 130.9012 84.6376) (end 134.2032 87.9396) (width 5) (layer "F.Cu") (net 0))
 (segment (start 129.0216 92.9688) (end 129.0216 96.6518) (width 5) (layer "F.Cu") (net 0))
 (segment (start 126.1514 87.7364) (end 126.1768 87.7364) (width 5) (layer "F.Cu") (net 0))
 (segment (start 133.142 110.6746) (end 145.142 110.6746) (width 5) (layer "F.Cu") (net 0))
 (segment (start 145.5062 107.015) (end 145.5062 106.0752) (width 5) (layer "F.Cu") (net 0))
 (segment (start 126.1768 87.7364) (end 126.253 87.8126) (width 5) (layer "F.Cu") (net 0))
 (segment (start 144.6934 114) (end 134 114) (width 6) (layer "F.Cu") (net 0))
 (segment (start 132.3998 59.771) (end 122.4176 69.7532) (width 6) (layer "F.Cu") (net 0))
 (segment (start 147.0556 59.771) (end 132.3998 59.771) (width 6) (layer "F.Cu") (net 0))
 (segment (start 137.094 76.1746) (end 133.954 76.1746) (width 5) (layer "F.Cu") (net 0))
 (segment (start 148.5034 78.948) (end 145.8054 76.25) (width 5) (layer "F.Cu") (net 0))
 (segment (start 133.142 103.1746) (end 133.142 110.6746) (width 5) (layer "F.Cu") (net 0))
 (segment (start 148.5034 85.3996) (end 148.5034 78.948) (width 5) (layer "F.Cu") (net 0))
 (segment (start 157.3172 84.7646) (end 157.3172 70.0326) (width 6) (layer "F.Cu") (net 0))
 (via (at 139.7 79.248) (size 1.3) (drill 0.9) (layers "F.Cu" "B.Cu") (free) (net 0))
 (via (at 145.7452 89.408) (size 1.3) (drill 0.9) (layers "F.Cu" "B.Cu") (free) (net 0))
 (via (at 134.0612 88.9) (size 1.3) (drill 0.9) (layers "F.Cu" "B.Cu") (free) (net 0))
 (via (at 132.08 78.232) (size 1.3) (drill 0.9) (layers "F.Cu" "B.Cu") (free) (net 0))
 (via (at 148.844 118.618) (size 1.3) (drill 0.9) (layers "F.Cu" "B.Cu") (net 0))
 (via (at 147.32 78.232) (size 1.3) (drill 0.9) (layers "F.Cu" "B.Cu") (free) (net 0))
 (segment (start 147.5232 91.5924) (end 144.3406 94.775) (width 0.6096) (layer "B.Cu") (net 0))
 (segment (start 148.162 79.119036) (end 148.162 78.6066) (width 0.6096) (layer "B.Cu") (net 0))
 (segment (start 148.162 78.6066) (end 147.462 77.9066) (width 0.6096) (layer "B.Cu") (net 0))
 (segment (start 134.954 89.3254) (end 134.2032 88.5746) (width 0.6096) (layer "B.Cu") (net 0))
 (segment (start 138.871564 77.019564) (end 139.7 77.848) (width 0.6096) (layer "B.Cu") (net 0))
 (segment (start 146.496 88.195564) (end 147.5232 89.222764) (width 0.6096) (layer "B.Cu") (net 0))
 (segment (start 134.954 89.787036) (end 134.954 89.3254) (width 0.6096) (layer "B.Cu") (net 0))
 (segment (start 133.604 87.376) (end 133.604 77.843564) (width 0.6096) (layer "B.Cu") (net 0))
 (segment (start 145.8976 77.741964) (end 146.62 77.019564) (width 0.6096) (layer "B.Cu") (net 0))
 (segment (start 145.238 89.7318) (end 145.8872 89.0826) (width 0.6096) (layer "B.Cu") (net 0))
 (segment (start 147.5232 89.222764) (end 147.5232 91.5924) (width 0.6096) (layer "B.Cu") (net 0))
 (segment (start 131.522 78.6066) (end 132.222 77.9066) (width 0.6096) (layer "B.Cu") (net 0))
 (segment (start 146.496 88.195564) (end 145.8976 87.597164) (width 0.6096) (layer "B.Cu") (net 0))
 (segment (start 140.528436 77.019564) (end 146.62 77.019564) (width 0.6096) (layer "B.Cu") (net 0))
 (segment (start 133.412 87.568) (end 133.604 87.376) (width 0.6096) (layer "B.Cu") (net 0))
 (segment (start 140.858 110.1646) (end 148.986 118.2926) (width 2) (layer "B.Cu") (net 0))
 (segment (start 132.78 77.019564) (end 138.871564 77.019564) (width 0.6096) (layer "B.Cu") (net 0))
 (segment (start 145.238 90.295036) (end 145.238 89.7318) (width 0.6096) (layer "B.Cu") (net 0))
 (segment (start 140.858 106.3546) (end 140.858 110.1646) (width 2) (layer "B.Cu") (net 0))
 (segment (start 139.842 80.3226) (end 139.842 78.9226) (width 0.6096) (layer "B.Cu") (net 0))
 (segment (start 133.604 77.843564) (end 132.78 77.019564) (width 0.6096) (layer "B.Cu") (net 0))
 (segment (start 131.522 79.119036) (end 131.522 78.6066) (width 0.6096) (layer "B.Cu") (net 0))
 (segment (start 139.7 77.848) (end 140.528436 77.019564) (width 0.6096) (layer "B.Cu") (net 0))
 (segment (start 145.8976 87.597164) (end 145.8976 77.741964) (width 0.6096) (layer "B.Cu") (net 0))
 (segment (start 144.3406 94.775) (end 140.716 94.775) (width 0.6096) (layer "B.Cu") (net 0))
 (segment (start 133.412 87.687564) (end 133.412 87.568) (width 0.6096) (layer "B.Cu") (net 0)))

